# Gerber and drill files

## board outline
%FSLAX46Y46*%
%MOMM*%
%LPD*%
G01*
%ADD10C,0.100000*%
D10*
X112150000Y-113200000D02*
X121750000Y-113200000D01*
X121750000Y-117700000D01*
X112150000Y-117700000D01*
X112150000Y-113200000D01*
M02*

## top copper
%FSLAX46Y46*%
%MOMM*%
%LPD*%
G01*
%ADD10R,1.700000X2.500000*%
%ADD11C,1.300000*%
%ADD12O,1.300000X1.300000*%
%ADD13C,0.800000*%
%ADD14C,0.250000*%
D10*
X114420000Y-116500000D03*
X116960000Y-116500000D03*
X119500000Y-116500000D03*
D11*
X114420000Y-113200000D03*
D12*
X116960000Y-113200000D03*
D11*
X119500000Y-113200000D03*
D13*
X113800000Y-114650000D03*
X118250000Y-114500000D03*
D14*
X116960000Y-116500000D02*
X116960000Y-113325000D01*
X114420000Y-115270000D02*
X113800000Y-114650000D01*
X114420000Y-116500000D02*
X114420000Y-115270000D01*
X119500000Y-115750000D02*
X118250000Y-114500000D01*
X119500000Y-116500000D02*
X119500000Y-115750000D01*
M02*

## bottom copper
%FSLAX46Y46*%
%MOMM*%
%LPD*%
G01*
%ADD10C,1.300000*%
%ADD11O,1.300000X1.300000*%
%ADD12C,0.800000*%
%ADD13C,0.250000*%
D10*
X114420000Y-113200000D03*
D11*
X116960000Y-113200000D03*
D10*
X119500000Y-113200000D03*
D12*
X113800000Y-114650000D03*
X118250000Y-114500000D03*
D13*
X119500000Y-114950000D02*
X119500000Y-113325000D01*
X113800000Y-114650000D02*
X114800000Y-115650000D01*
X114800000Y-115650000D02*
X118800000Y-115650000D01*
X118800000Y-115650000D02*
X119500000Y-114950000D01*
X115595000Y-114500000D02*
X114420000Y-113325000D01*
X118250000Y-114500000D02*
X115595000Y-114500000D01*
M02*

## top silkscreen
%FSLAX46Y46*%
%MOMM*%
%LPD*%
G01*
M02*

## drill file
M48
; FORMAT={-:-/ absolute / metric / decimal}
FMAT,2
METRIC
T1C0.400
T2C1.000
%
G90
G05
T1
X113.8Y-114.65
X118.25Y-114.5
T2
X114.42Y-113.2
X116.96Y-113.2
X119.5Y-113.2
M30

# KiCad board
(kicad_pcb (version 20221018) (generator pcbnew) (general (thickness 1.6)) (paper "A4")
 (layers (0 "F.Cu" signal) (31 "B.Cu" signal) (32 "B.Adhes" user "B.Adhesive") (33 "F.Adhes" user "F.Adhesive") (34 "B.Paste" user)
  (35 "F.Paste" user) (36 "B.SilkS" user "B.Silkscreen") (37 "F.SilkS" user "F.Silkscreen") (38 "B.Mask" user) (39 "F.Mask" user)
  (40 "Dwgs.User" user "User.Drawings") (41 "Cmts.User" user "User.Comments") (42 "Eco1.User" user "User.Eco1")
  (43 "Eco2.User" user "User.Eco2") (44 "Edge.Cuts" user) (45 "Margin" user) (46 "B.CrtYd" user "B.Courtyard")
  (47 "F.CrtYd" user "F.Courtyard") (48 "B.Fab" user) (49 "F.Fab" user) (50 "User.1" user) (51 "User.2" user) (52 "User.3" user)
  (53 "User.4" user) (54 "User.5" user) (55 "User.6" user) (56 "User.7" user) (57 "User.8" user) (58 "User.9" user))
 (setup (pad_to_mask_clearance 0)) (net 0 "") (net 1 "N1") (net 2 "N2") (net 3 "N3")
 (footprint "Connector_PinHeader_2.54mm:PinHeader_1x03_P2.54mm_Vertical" (layer "F.Cu") (at 114.42 116.5 90)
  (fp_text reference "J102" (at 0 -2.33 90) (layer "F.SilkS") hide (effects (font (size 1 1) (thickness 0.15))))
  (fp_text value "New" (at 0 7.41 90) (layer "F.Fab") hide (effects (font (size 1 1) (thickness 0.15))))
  (pad "1" smd rect (at 0 0 90) (size 2.5 1.7) (layers "F.Cu" "F.Paste" "F.Mask") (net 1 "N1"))
  (pad "2" smd rect (at 0 2.54 90) (size 2.5 1.7) (layers "F.Cu" "F.Paste" "F.Mask") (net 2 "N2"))
  (pad "3" smd rect (at 0 5.08 90) (size 2.5 1.7) (layers "F.Cu" "F.Paste" "F.Mask") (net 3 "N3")))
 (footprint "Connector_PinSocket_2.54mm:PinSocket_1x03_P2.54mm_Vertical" (layer "F.Cu") (at 114.42 113.2 90)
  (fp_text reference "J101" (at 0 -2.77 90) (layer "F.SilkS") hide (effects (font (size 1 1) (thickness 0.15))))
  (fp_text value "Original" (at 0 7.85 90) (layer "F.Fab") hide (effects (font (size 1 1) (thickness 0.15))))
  (pad "1" thru_hole circle (at 0 0 90) (size 1.3 1.3) (drill 1) (layers "*.Cu" "*.Mask") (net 3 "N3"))
  (pad "2" thru_hole oval (at 0 2.54 90) (size 1.3 1.3) (drill 1) (layers "*.Cu" "*.Mask") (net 2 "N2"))
  (pad "3" thru_hole circle (at 0 5.08 90) (size 1.3 1.3) (drill 1) (layers "*.Cu" "*.Mask") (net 1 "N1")))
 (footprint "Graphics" (layer "B.Cu") (at 116.95 115.65 -135)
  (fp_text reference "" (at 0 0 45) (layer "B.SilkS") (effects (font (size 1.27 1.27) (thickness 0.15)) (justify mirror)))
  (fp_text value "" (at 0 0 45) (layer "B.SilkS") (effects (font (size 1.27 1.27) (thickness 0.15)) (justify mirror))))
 (gr_rect (start 112.15 113.2) (end 121.75 117.7) (stroke (width 0.1) (type default)) (fill none) (layer "Edge.Cuts"))
 (segment (start 116.96 116.5) (end 116.96 113.325) (width 0.25) (layer "F.Cu") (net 2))
 (segment (start 114.42 115.27) (end 113.8 114.65) (width 0.25) (layer "F.Cu") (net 1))
 (segment (start 114.42 116.5) (end 114.42 115.27) (width 0.25) (layer "F.Cu") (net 1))
 (via (at 113.8 114.65) (size 0.8) (drill 0.4) (layers "F.Cu" "B.Cu") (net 1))
 (segment (start 119.5 114.95) (end 119.5 113.325) (width 0.25) (layer "B.Cu") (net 1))
 (segment (start 113.8 114.65) (end 114.8 115.65) (width 0.25) (layer "B.Cu") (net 1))
 (segment (start 114.8 115.65) (end 118.8 115.65) (width 0.25) (layer "B.Cu") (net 1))
 (segment (start 118.8 115.65) (end 119.5 114.95) (width 0.25) (layer "B.Cu") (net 1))
 (segment (start 119.5 115.75) (end 118.25 114.5) (width 0.25) (layer "F.Cu") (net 3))
 (segment (start 119.5 116.5) (end 119.5 115.75) (width 0.25) (layer "F.Cu") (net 3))
 (via (at 118.25 114.5) (size 0.8) (drill 0.4) (layers "F.Cu" "B.Cu") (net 3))
 (segment (start 115.595 114.5) (end 114.42 113.325) (width 0.25) (layer "B.Cu") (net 3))
 (segment (start 118.25 114.5) (end 115.595 114.5) (width 0.25) (layer "B.Cu") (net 3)))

